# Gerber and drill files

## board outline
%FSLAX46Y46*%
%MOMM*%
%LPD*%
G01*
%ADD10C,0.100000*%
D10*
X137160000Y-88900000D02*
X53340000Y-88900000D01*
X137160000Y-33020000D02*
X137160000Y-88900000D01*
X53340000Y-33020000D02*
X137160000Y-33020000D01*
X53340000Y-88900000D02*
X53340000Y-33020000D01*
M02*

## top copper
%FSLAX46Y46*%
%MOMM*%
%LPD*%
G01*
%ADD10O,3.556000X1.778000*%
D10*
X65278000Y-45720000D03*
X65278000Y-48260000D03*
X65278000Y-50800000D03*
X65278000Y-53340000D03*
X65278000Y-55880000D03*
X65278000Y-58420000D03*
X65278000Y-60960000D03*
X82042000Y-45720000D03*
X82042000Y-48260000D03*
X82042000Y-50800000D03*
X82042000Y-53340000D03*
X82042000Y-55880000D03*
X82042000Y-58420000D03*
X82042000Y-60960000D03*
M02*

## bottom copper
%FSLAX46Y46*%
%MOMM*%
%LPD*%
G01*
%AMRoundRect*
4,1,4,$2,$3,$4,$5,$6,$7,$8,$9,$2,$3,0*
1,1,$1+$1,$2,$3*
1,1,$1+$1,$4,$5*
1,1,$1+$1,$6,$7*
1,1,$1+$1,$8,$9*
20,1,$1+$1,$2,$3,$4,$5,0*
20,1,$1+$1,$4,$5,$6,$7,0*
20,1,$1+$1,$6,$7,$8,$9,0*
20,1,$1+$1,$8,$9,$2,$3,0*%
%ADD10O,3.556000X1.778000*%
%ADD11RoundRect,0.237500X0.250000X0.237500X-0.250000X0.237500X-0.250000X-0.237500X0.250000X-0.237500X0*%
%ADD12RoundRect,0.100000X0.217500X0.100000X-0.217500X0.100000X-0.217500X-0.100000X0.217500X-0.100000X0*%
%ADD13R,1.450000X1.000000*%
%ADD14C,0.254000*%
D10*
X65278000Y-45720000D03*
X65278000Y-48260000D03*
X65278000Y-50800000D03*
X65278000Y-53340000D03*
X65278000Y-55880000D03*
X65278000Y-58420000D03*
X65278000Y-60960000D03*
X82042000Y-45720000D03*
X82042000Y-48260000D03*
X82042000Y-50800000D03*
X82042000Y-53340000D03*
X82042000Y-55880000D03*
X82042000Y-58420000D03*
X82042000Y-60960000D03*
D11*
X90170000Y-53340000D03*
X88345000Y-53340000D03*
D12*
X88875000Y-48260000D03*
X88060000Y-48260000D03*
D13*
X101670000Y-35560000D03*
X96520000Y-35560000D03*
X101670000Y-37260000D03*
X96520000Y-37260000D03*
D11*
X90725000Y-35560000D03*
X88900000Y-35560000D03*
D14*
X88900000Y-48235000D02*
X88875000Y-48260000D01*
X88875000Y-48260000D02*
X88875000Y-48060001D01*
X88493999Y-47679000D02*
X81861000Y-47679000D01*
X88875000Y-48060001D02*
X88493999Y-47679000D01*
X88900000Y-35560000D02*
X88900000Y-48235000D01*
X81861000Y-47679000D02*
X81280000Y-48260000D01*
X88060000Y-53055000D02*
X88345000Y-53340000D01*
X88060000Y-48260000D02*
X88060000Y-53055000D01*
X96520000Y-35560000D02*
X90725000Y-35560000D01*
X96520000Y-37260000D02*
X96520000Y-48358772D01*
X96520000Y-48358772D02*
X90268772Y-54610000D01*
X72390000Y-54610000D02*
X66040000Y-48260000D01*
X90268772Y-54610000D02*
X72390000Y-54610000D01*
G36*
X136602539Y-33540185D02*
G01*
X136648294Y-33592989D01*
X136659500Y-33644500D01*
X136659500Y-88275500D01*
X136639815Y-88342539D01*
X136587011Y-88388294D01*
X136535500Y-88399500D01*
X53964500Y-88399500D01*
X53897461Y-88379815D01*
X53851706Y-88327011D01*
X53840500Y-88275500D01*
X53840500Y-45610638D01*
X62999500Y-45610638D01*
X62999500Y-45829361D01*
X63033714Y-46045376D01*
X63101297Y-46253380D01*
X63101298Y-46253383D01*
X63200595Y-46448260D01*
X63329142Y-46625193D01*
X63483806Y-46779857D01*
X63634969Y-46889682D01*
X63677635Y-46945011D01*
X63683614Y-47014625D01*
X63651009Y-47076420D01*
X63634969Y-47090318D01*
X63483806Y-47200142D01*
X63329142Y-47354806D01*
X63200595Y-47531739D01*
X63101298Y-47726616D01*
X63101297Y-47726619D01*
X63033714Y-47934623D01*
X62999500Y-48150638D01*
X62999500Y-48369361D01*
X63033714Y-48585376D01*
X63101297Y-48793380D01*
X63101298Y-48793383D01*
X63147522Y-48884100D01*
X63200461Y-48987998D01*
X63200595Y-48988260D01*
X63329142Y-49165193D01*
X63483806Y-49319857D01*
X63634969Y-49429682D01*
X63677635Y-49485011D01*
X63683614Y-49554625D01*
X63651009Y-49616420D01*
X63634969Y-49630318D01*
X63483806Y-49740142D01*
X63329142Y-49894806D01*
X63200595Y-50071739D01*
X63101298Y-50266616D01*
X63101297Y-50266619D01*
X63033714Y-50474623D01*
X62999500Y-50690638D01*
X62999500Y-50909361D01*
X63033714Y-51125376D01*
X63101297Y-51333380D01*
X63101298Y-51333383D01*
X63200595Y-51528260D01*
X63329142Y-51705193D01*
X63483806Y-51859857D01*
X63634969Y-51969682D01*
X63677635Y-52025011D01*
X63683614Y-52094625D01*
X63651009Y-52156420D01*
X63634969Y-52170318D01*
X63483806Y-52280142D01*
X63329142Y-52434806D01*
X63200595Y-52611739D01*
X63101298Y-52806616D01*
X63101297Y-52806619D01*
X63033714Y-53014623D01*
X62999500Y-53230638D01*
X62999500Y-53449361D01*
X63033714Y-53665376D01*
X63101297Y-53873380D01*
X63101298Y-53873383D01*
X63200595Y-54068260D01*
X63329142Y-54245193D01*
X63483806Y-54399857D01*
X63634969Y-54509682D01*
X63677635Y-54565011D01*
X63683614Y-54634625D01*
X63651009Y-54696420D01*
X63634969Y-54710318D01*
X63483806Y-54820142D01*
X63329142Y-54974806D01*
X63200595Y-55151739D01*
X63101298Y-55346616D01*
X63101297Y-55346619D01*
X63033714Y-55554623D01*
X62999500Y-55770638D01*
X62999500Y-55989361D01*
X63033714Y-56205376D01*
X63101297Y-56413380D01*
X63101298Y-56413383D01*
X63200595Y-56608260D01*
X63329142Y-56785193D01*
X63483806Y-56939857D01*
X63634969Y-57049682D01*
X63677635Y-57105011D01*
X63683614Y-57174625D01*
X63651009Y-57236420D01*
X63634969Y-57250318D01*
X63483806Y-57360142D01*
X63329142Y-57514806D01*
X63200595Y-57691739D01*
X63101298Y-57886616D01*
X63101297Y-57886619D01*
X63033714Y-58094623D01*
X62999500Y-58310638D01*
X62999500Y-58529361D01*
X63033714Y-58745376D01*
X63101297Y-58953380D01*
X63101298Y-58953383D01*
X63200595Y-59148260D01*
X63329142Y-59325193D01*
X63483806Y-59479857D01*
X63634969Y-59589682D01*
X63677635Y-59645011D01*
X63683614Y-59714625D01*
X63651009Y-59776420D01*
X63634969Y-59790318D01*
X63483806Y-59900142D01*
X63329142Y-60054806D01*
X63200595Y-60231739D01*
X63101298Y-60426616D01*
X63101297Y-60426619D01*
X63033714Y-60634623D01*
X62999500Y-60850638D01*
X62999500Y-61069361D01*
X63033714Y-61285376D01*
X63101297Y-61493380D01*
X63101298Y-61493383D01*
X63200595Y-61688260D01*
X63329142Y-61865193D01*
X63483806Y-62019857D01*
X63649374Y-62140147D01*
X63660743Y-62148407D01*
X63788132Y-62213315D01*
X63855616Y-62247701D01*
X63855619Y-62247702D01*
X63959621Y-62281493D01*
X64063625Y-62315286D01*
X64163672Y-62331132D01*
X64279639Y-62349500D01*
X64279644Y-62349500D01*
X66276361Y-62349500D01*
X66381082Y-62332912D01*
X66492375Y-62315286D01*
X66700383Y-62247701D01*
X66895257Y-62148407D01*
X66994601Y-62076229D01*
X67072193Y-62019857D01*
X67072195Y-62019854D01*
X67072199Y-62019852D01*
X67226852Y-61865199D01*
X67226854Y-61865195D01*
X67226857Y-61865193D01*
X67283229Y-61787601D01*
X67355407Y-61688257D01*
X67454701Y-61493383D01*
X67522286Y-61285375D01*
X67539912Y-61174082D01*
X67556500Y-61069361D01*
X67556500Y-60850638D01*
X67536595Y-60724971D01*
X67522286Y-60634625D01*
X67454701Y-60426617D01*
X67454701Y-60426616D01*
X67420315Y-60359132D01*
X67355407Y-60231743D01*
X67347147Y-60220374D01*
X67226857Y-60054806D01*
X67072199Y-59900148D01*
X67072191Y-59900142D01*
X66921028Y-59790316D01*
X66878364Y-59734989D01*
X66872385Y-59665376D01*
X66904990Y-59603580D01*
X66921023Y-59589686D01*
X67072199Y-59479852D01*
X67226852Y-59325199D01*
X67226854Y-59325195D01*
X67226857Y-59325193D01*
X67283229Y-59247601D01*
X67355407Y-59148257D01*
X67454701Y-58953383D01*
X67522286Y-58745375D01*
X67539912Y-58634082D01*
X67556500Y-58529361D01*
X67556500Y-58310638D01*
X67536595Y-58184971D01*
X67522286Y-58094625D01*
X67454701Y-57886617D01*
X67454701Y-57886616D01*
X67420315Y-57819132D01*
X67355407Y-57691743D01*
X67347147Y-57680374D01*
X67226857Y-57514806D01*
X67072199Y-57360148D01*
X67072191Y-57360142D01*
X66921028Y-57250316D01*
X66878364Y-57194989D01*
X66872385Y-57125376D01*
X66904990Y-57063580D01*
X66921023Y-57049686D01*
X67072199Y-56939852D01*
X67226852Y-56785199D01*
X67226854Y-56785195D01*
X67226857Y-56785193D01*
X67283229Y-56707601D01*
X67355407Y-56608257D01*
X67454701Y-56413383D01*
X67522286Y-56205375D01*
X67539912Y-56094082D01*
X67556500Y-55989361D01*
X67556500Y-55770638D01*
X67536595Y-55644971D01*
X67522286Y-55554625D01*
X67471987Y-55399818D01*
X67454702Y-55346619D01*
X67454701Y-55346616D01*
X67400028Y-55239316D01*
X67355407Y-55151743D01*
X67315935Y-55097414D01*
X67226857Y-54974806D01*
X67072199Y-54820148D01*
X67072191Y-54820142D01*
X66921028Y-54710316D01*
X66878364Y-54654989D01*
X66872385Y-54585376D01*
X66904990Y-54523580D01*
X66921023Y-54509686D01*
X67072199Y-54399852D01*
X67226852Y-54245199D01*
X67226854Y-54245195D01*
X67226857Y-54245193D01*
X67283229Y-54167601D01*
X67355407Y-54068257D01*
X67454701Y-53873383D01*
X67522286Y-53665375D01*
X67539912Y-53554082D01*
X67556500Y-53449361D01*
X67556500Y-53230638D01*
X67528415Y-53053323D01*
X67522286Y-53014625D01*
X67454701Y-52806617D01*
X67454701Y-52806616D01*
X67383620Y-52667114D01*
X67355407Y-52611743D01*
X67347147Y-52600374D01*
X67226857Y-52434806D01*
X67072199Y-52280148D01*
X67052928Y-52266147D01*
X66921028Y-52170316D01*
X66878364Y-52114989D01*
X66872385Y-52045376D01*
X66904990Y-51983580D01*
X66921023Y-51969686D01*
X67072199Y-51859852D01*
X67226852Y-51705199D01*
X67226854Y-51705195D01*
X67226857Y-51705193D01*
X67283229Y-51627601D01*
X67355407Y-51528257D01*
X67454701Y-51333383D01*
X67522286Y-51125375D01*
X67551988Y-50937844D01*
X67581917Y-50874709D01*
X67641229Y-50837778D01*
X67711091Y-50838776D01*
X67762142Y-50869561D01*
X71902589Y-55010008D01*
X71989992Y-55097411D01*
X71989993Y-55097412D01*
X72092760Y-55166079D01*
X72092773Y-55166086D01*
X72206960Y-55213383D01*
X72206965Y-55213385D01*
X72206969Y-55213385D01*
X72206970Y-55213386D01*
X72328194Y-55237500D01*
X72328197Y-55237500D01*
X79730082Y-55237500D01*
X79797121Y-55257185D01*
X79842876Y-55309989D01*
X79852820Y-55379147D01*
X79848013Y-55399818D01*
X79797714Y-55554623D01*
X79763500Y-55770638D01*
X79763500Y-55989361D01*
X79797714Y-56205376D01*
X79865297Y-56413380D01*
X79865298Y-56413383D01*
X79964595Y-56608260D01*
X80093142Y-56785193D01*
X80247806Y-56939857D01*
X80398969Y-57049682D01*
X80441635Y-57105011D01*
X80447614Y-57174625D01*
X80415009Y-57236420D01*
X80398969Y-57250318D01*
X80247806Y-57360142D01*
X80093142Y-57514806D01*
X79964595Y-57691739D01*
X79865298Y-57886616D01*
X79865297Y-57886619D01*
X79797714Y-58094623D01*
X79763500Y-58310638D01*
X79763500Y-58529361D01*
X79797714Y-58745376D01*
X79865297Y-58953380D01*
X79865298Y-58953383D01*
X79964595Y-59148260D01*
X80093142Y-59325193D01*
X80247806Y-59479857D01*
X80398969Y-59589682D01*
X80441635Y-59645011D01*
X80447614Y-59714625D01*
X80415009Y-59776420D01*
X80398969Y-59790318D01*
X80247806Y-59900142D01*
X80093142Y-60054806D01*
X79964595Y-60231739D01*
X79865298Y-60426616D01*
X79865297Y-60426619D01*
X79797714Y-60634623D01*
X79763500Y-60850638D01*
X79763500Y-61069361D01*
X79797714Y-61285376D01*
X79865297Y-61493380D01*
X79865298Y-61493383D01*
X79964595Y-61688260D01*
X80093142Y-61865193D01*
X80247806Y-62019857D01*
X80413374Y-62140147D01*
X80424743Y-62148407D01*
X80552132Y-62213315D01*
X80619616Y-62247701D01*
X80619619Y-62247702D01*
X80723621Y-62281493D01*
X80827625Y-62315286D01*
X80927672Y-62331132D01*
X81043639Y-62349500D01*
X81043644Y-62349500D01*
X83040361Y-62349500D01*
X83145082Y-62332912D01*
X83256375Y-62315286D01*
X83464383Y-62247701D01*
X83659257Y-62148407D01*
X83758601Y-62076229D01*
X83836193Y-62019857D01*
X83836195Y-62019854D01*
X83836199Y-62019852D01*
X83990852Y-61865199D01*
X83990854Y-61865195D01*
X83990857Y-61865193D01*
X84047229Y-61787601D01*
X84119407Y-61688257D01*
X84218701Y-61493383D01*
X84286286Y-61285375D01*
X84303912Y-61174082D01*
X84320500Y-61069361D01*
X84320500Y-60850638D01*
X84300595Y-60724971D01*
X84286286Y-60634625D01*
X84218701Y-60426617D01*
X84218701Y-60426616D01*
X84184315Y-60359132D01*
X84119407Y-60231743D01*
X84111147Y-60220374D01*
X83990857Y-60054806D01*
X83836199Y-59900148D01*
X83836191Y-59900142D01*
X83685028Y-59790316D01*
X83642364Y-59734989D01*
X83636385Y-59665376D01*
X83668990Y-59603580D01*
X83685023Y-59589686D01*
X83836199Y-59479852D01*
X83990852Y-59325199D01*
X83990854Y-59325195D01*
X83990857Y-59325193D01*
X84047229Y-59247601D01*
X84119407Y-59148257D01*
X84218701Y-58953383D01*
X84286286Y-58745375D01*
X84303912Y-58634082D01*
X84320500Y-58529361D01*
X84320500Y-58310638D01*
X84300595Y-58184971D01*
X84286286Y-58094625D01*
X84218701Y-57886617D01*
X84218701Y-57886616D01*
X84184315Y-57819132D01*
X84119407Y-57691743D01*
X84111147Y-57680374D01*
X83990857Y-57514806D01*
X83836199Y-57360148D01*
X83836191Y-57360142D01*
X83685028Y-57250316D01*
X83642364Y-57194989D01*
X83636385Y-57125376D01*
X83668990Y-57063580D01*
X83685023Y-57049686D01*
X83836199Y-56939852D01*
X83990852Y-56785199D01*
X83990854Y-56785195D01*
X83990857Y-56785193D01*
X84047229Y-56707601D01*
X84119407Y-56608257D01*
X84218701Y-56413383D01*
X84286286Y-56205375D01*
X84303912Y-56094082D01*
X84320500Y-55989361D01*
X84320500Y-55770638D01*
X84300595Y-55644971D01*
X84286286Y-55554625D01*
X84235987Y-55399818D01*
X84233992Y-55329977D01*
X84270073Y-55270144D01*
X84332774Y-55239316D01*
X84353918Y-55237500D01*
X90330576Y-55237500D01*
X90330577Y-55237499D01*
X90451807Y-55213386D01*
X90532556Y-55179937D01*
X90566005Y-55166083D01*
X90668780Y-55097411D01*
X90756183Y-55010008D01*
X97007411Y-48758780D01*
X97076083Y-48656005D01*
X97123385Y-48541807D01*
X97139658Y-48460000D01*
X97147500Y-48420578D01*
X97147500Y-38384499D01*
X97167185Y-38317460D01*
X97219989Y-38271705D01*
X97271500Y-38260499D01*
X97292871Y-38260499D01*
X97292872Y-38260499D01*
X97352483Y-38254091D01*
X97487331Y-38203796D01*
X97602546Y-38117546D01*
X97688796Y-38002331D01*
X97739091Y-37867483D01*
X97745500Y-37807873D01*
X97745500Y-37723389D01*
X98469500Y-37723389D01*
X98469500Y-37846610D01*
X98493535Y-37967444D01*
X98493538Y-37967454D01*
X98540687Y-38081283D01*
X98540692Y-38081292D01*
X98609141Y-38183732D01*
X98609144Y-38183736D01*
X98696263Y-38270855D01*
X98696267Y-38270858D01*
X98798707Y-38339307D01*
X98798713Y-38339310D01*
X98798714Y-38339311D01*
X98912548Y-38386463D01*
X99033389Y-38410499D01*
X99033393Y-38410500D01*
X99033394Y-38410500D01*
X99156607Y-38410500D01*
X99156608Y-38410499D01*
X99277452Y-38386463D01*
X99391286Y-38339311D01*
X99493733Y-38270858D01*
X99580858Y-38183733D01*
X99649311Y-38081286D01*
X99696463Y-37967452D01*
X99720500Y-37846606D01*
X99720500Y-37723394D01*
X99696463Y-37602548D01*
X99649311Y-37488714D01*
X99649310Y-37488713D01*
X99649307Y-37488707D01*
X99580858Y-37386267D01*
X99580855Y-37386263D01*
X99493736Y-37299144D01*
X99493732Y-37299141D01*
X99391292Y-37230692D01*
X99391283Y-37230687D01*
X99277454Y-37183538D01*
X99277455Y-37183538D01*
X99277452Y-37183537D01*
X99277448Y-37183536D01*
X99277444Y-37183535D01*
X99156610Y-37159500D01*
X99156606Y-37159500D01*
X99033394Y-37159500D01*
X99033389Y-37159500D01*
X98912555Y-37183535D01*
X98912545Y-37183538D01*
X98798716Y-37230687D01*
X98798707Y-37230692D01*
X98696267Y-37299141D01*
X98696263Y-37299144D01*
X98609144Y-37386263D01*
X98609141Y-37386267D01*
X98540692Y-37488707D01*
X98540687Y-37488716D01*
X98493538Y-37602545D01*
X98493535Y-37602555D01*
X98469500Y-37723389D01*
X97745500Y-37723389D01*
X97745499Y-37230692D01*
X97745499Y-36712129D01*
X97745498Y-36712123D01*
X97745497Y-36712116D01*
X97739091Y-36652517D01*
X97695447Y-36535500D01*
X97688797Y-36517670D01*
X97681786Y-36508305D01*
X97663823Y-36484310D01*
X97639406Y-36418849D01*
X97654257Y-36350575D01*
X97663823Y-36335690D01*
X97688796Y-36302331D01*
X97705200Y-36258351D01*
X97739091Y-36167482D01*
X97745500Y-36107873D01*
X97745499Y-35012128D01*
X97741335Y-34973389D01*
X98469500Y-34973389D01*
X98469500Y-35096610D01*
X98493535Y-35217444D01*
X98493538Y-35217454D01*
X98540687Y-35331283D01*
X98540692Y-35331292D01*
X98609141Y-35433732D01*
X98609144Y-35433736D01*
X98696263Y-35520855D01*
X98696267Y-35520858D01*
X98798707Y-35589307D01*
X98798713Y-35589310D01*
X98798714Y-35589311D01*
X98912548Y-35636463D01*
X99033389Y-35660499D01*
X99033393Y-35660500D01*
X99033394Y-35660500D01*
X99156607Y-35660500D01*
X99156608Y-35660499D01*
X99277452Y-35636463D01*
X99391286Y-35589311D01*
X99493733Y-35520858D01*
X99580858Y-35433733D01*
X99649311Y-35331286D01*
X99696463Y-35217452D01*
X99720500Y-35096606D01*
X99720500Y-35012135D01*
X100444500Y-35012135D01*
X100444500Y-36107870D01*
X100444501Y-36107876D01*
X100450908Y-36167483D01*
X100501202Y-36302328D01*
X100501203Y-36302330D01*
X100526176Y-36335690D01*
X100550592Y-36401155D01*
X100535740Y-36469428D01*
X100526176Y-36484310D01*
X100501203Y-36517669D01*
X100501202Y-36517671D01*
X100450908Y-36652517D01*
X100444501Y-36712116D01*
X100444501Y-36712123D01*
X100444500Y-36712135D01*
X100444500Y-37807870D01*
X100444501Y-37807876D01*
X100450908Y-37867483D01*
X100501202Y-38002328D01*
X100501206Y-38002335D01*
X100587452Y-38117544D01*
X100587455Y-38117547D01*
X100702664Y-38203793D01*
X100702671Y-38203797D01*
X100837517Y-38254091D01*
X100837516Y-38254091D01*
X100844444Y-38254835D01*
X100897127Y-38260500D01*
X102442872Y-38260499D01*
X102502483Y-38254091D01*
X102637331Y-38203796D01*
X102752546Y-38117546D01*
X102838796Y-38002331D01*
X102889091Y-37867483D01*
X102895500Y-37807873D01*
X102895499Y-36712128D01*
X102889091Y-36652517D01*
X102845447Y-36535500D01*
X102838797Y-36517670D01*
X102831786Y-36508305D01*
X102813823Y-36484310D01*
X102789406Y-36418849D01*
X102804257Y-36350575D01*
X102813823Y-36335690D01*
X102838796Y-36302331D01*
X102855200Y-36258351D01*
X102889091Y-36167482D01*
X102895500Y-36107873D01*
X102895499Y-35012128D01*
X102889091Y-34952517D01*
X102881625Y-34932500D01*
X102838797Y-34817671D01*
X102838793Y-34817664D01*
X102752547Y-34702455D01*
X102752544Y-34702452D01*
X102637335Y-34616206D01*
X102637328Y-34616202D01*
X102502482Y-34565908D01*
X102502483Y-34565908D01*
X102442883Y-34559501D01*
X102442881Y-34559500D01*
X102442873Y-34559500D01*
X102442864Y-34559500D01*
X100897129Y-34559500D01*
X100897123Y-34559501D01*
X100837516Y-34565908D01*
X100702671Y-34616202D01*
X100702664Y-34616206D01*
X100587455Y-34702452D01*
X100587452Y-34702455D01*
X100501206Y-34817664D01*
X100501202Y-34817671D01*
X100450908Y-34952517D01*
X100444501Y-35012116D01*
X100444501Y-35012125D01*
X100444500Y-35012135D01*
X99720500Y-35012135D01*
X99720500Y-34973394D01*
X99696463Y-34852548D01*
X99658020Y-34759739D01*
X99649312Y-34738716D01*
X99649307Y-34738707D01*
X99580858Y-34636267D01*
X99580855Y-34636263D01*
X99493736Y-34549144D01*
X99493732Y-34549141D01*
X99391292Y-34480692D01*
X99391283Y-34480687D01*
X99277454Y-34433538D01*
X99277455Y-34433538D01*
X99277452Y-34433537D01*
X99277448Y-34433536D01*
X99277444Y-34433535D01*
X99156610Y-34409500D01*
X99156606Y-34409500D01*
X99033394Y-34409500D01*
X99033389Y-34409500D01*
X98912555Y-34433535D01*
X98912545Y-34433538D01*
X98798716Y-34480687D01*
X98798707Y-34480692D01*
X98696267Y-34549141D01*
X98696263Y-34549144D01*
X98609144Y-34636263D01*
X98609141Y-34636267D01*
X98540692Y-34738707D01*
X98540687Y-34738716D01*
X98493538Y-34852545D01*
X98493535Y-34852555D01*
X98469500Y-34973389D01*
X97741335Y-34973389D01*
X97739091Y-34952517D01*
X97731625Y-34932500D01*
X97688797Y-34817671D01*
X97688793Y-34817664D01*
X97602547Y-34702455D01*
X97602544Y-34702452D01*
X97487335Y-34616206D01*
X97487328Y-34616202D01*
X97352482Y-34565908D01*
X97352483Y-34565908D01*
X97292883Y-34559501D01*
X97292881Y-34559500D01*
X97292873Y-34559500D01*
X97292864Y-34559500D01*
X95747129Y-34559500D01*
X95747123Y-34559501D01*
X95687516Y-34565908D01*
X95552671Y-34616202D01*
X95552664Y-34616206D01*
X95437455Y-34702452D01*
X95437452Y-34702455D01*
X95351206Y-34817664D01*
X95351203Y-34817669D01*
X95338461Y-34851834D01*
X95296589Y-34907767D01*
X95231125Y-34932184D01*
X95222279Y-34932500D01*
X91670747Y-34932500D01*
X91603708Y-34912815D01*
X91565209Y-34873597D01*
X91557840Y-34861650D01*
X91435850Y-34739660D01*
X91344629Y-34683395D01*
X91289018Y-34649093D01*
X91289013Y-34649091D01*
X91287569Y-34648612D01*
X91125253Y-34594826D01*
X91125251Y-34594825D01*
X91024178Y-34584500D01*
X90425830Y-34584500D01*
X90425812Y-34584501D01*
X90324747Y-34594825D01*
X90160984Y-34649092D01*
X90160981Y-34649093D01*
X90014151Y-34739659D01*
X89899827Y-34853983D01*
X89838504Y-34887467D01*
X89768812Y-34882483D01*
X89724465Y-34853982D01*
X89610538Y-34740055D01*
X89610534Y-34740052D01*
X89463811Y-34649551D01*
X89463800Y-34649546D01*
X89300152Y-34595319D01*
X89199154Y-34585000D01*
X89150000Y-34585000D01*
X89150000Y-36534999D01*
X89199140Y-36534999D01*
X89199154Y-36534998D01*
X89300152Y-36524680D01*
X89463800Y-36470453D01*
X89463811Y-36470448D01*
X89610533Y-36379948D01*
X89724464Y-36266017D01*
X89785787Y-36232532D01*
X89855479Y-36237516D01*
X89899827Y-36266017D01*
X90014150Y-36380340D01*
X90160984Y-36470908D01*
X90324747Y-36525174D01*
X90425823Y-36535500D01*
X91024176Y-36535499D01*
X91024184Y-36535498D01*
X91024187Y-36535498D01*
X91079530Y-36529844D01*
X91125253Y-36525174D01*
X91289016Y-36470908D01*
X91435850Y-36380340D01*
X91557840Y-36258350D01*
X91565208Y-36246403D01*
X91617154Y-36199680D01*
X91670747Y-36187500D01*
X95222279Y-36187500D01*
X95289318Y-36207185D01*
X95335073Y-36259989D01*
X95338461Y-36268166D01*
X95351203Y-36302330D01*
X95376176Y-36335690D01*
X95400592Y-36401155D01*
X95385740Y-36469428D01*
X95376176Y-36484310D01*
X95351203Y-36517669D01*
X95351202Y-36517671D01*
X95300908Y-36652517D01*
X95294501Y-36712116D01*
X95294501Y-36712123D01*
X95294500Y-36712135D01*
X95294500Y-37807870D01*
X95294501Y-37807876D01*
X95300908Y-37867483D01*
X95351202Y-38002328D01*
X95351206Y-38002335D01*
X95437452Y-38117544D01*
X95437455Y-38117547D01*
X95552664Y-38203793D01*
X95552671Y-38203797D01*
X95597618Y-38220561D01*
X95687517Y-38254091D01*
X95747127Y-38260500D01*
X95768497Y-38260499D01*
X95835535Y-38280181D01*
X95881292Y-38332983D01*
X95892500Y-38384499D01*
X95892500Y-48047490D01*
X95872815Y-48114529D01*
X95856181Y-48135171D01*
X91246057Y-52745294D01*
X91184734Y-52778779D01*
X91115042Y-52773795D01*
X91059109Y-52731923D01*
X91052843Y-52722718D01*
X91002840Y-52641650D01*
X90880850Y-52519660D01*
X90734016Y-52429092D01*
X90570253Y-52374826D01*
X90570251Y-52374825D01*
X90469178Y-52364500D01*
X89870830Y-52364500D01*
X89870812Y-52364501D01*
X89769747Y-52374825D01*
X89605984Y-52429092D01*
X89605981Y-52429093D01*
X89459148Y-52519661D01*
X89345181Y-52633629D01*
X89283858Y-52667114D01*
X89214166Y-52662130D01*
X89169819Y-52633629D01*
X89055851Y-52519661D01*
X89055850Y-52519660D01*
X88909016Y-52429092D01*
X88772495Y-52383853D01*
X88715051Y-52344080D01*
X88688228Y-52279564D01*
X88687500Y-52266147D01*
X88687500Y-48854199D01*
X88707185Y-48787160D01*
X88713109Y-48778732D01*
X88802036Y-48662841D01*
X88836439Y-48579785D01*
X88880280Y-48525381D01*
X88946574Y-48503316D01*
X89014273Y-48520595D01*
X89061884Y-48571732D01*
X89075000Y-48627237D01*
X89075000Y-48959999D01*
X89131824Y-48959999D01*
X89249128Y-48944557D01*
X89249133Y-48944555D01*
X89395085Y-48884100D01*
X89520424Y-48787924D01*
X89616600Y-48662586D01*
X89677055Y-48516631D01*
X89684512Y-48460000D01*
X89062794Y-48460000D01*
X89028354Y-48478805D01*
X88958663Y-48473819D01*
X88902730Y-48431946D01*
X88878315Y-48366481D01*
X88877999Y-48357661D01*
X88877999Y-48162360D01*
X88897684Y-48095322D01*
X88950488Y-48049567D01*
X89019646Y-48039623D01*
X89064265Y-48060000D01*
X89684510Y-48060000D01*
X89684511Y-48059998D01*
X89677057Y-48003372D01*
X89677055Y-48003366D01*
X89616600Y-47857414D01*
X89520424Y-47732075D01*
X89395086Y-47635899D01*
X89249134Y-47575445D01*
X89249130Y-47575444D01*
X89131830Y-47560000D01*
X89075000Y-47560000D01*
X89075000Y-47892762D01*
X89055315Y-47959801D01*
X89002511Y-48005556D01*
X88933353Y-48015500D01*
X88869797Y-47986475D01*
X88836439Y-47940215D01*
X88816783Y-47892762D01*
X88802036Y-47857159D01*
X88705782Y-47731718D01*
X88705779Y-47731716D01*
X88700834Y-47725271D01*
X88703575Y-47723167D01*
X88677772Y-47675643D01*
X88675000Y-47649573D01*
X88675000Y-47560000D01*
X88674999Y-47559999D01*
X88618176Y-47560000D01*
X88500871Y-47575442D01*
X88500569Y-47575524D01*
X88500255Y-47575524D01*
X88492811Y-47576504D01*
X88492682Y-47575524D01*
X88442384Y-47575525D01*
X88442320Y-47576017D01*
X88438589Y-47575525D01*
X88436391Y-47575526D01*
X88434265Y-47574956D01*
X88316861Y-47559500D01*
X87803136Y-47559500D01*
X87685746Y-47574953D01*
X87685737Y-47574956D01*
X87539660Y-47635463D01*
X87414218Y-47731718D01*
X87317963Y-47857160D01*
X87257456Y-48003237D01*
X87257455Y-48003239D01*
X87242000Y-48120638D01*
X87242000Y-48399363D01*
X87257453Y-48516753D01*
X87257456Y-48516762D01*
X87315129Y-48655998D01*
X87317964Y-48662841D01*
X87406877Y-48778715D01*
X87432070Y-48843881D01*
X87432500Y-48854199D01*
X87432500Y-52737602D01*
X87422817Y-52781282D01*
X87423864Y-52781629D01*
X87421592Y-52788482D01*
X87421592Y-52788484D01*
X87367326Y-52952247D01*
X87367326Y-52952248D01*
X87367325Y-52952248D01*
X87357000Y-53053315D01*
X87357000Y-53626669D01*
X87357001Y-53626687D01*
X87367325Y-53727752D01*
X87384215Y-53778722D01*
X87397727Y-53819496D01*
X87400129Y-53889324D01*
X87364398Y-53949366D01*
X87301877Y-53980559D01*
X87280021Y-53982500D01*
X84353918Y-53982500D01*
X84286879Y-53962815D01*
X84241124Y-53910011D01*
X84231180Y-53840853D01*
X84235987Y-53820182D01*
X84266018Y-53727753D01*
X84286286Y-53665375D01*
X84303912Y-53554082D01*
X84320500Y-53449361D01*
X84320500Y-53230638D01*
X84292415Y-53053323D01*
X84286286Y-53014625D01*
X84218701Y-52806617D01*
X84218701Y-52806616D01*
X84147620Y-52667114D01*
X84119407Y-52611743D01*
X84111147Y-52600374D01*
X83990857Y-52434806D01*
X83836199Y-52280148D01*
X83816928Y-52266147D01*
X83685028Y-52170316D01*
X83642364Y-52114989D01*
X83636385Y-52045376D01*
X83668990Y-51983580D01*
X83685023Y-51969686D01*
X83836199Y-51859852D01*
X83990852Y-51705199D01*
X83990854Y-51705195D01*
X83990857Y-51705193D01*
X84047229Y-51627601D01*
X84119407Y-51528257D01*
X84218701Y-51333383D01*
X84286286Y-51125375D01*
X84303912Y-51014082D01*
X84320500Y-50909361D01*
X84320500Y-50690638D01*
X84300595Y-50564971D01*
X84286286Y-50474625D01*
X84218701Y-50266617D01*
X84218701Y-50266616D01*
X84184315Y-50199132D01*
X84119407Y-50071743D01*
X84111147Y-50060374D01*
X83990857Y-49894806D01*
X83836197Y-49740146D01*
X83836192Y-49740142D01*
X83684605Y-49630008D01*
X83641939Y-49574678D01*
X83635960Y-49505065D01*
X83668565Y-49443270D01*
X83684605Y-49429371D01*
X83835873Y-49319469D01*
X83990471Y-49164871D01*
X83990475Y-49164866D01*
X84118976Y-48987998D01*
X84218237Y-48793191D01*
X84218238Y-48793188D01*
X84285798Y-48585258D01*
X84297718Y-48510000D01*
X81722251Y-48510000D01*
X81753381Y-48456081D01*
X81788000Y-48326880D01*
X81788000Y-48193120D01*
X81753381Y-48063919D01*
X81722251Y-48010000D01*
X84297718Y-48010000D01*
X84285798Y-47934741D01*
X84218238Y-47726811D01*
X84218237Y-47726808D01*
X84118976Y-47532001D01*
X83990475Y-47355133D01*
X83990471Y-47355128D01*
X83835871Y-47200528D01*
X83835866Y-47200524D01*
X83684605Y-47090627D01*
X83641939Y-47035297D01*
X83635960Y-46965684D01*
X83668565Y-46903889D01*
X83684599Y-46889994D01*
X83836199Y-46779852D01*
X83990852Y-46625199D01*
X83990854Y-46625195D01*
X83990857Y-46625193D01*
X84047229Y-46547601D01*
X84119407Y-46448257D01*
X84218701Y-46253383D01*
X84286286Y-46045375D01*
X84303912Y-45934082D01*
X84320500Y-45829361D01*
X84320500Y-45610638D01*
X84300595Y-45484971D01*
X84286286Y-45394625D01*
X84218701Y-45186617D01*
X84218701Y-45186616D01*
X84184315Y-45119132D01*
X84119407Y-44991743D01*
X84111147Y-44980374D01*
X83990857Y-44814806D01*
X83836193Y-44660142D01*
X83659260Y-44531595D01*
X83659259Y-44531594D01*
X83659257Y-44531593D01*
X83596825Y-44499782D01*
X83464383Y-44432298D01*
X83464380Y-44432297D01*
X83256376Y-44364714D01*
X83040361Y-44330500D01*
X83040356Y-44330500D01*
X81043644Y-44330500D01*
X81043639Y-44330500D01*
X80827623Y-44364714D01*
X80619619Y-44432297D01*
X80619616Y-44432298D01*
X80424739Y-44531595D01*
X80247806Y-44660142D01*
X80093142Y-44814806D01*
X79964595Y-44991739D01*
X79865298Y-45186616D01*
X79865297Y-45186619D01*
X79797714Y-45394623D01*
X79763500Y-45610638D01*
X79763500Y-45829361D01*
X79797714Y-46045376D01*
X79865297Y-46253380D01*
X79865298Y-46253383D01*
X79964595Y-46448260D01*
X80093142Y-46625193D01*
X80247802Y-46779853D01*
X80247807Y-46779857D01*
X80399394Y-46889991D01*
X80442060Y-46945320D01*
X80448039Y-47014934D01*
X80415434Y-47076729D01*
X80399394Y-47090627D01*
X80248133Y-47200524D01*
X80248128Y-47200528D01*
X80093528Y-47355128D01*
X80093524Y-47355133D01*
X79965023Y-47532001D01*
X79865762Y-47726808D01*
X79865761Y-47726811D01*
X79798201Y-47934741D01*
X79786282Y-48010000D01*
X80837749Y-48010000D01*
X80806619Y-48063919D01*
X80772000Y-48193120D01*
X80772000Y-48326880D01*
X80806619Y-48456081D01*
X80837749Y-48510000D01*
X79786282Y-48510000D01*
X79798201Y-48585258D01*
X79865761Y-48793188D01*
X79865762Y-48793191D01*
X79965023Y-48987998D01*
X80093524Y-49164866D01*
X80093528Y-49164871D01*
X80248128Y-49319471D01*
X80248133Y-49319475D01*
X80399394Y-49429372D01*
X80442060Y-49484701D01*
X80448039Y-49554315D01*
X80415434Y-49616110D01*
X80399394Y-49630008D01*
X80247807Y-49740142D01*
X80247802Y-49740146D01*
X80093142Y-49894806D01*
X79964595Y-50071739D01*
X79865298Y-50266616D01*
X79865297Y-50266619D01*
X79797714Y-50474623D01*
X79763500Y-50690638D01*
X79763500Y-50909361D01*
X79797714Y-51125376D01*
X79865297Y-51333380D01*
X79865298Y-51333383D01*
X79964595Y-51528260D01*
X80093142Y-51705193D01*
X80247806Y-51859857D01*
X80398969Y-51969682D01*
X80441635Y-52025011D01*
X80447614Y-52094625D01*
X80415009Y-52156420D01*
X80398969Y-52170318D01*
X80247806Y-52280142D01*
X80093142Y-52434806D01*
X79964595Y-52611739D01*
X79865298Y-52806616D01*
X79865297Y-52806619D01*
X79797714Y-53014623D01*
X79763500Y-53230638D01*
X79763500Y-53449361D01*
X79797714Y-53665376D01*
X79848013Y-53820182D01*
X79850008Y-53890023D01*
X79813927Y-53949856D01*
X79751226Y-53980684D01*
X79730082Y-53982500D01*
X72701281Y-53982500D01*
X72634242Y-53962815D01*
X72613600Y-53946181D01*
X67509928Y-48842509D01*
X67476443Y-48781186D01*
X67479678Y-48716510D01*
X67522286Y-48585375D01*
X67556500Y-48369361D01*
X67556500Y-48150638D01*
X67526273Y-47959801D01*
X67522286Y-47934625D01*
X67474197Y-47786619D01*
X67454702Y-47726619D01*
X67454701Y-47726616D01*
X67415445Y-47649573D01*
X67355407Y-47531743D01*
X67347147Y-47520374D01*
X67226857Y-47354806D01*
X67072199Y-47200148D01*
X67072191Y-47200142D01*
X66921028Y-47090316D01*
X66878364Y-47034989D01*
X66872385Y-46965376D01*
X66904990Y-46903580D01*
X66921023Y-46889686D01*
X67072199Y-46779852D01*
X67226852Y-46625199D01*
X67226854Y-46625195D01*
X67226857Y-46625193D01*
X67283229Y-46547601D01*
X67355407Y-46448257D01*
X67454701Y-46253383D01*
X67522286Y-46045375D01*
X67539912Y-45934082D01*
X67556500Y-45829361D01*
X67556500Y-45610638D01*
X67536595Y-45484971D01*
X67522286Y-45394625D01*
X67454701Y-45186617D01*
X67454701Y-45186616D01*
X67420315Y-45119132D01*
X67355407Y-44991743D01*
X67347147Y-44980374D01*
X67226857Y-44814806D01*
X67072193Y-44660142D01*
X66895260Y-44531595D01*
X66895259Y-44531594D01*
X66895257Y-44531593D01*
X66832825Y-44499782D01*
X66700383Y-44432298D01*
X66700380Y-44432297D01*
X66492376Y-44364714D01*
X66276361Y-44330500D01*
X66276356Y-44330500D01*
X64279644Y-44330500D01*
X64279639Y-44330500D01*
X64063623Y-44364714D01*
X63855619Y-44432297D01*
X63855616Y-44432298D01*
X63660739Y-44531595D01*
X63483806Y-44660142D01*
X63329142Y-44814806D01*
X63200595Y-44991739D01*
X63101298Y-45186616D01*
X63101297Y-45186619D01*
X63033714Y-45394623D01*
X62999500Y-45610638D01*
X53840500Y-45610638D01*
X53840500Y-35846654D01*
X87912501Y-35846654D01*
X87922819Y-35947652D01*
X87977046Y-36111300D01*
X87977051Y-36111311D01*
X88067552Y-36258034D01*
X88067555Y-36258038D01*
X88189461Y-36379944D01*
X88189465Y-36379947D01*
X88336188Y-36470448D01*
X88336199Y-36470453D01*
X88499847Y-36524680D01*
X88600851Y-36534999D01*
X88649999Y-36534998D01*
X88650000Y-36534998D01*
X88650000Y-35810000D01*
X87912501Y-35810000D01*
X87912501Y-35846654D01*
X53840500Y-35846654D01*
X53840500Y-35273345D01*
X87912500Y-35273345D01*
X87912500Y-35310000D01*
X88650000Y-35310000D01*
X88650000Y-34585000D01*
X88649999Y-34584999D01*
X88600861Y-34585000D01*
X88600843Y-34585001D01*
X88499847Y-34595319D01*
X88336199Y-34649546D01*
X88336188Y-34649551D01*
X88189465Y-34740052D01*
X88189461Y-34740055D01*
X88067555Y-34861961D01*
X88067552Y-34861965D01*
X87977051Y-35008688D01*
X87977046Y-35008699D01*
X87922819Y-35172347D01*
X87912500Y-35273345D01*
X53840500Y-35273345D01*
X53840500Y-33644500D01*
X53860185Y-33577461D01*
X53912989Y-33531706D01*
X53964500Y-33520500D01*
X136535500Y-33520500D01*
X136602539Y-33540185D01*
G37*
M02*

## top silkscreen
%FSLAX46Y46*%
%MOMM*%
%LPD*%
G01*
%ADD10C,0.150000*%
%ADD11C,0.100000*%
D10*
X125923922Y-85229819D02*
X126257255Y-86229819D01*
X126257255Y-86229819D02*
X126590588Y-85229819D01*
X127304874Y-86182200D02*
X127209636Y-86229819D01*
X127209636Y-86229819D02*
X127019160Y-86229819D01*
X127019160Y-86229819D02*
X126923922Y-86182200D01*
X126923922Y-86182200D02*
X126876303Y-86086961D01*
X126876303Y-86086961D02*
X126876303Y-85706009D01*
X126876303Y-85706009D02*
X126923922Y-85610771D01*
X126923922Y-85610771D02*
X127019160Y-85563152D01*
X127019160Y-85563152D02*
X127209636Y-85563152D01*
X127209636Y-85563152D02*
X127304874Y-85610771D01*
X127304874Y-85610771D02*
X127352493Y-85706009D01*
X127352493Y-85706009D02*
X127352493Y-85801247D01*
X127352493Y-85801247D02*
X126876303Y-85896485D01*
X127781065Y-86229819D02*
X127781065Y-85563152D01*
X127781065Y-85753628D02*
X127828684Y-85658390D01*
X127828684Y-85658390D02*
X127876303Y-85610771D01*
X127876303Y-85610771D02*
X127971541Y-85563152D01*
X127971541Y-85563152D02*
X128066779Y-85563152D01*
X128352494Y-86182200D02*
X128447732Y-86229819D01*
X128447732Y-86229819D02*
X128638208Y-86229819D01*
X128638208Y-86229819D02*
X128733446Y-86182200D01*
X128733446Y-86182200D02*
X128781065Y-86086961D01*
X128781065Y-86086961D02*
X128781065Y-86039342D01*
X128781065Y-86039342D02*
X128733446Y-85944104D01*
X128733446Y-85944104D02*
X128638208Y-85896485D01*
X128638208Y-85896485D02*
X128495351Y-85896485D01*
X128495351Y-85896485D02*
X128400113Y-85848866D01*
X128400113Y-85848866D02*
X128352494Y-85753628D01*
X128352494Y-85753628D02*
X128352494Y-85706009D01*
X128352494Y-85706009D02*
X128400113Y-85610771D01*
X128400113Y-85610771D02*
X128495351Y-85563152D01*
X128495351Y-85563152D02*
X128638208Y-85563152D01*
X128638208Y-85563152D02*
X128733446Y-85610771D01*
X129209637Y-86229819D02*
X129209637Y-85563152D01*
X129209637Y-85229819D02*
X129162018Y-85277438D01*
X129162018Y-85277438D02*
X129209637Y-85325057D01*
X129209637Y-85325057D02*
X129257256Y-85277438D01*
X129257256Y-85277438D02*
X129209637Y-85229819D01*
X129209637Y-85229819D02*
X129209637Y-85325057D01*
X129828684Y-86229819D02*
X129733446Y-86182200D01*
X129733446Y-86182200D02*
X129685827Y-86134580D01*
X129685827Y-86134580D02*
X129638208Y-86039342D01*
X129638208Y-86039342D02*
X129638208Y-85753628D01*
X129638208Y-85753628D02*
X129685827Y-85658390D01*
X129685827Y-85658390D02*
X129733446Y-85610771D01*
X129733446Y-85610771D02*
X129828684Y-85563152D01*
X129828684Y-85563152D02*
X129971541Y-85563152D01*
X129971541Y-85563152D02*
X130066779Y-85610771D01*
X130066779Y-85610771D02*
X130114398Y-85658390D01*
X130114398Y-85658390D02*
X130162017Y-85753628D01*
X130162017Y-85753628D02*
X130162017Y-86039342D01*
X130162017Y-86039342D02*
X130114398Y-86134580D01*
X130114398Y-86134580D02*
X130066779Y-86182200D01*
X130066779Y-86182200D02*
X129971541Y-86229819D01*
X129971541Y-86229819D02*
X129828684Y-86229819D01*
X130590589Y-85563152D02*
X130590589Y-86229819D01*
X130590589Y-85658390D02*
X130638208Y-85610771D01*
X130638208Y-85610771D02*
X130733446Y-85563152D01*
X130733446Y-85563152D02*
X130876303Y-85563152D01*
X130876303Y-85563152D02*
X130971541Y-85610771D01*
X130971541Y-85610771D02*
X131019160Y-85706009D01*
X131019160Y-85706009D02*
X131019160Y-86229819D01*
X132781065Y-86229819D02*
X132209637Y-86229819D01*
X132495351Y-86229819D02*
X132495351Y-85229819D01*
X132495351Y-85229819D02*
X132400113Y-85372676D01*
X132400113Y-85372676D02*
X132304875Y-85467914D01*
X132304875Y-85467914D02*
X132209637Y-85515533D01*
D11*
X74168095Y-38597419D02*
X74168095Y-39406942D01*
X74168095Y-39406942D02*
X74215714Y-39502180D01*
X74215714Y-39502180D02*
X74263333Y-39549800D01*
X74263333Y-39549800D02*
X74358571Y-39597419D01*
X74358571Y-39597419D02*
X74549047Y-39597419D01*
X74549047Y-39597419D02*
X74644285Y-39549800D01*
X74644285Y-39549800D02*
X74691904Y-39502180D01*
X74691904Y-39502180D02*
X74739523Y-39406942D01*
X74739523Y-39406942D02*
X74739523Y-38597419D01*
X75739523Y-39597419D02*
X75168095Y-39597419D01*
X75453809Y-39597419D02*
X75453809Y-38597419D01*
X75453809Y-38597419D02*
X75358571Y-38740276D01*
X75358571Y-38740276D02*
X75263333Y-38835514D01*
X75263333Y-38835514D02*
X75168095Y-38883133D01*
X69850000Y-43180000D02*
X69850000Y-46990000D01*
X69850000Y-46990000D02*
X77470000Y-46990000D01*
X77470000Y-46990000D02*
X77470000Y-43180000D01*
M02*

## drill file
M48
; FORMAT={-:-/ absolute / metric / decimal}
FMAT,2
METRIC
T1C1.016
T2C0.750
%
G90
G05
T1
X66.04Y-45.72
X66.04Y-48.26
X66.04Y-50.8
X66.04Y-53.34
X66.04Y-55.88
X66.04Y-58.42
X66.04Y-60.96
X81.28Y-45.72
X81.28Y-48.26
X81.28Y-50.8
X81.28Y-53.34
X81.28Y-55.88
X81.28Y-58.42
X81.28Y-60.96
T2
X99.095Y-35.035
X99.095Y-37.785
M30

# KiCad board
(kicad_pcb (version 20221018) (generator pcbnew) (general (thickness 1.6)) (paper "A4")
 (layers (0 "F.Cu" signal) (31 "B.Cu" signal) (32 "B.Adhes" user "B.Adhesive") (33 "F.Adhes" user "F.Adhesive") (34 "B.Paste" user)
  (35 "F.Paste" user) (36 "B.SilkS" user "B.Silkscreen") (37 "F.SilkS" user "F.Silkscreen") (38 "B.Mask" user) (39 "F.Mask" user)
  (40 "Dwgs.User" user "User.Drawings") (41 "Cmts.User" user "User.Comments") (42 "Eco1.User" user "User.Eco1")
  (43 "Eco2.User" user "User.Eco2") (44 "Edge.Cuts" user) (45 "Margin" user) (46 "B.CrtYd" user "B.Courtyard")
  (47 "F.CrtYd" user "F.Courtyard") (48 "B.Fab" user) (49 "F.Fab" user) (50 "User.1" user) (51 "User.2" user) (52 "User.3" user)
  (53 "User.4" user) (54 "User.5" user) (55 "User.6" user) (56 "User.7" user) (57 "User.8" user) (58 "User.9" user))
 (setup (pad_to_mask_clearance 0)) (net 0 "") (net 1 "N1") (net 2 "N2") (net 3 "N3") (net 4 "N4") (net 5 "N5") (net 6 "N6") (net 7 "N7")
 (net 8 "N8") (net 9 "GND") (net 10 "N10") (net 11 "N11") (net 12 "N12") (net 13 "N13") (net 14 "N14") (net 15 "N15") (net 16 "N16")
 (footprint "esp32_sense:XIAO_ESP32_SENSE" (layer "F.Cu") (at 73.66 53.34)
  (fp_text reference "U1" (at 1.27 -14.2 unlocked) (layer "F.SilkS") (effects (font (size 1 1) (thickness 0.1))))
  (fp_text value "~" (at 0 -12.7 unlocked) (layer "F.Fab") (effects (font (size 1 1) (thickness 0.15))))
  (fp_line (start -3.81 -10.16) (end -3.81 -6.35) (stroke (width 0.1) (type default)) (layer "F.SilkS"))
  (fp_line (start -3.81 -6.35) (end 3.81 -6.35) (stroke (width 0.1) (type default)) (layer "F.SilkS"))
  (fp_line (start 3.81 -6.35) (end 3.81 -10.16) (stroke (width 0.1) (type default)) (layer "F.SilkS"))
  (pad "1" thru_hole oval (at -7.62 -7.62) (size 3.556 1.778) (drill 1.016 (offset -0.762 0)) (layers "*.Cu" "*.Mask") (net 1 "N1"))
  (pad "2" thru_hole oval (at -7.62 -5.08) (size 3.556 1.778) (drill 1.016 (offset -0.762 0)) (layers "*.Cu" "*.Mask") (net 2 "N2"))
  (pad "3" thru_hole oval (at -7.62 -2.54) (size 3.556 1.778) (drill 1.016 (offset -0.762 0)) (layers "*.Cu" "*.Mask") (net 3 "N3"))
  (pad "4" thru_hole oval (at -7.62 0) (size 3.556 1.778) (drill 1.016 (offset -0.762 0)) (layers "*.Cu" "*.Mask") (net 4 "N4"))
  (pad "5" thru_hole oval (at -7.62 2.54) (size 3.556 1.778) (drill 1.016 (offset -0.762 0)) (layers "*.Cu" "*.Mask") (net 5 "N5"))
  (pad "6" thru_hole oval (at -7.62 5.08) (size 3.556 1.778) (drill 1.016 (offset -0.762 0)) (layers "*.Cu" "*.Mask") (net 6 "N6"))
  (pad "7" thru_hole oval (at -7.62 7.62) (size 3.556 1.778) (drill 1.016 (offset -0.762 0)) (layers "*.Cu" "*.Mask") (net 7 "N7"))
  (pad "8" thru_hole oval (at 7.62 -7.62) (size 3.556 1.778) (drill 1.016 (offset 0.762 0)) (layers "*.Cu" "*.Mask") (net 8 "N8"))
  (pad "9" thru_hole oval (at 7.62 -5.08) (size 3.556 1.778) (drill 1.016 (offset 0.762 0)) (layers "*.Cu" "*.Mask") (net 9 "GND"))
  (pad "10" thru_hole oval (at 7.62 -2.54) (size 3.556 1.778) (drill 1.016 (offset 0.762 0)) (layers "*.Cu" "*.Mask") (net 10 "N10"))
  (pad "11" thru_hole oval (at 7.62 0) (size 3.556 1.778) (drill 1.016 (offset 0.762 0)) (layers "*.Cu" "*.Mask") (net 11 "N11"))
  (pad "12" thru_hole oval (at 7.62 2.54) (size 3.556 1.778) (drill 1.016 (offset 0.762 0)) (layers "*.Cu" "*.Mask") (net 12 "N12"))
  (pad "13" thru_hole oval (at 7.62 5.08) (size 3.556 1.778) (drill 1.016 (offset 0.762 0)) (layers "*.Cu" "*.Mask") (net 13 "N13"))
  (pad "14" thru_hole oval (at 7.62 7.62) (size 3.556 1.778) (drill 1.016 (offset 0.762 0)) (layers "*.Cu" "*.Mask") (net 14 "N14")))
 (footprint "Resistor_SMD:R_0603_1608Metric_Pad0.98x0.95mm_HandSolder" (layer "B.Cu") (at 89.2575 53.34 180)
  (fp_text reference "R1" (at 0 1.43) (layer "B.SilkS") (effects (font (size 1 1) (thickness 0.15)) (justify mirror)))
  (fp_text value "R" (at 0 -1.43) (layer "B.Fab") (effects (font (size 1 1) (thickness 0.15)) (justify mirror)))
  (pad "1" smd roundrect (at -0.9125 0 180) (size 0.975 0.95) (layers "B.Cu" "B.Paste" "B.Mask") (roundrect_rratio 0.25) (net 11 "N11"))
  (pad "2" smd roundrect (at 0.9125 0 180) (size 0.975 0.95) (layers "B.Cu" "B.Paste" "B.Mask") (roundrect_rratio 0.25) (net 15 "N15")))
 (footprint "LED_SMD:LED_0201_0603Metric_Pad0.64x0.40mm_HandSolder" (layer "B.Cu") (at 88.4675 48.26 180)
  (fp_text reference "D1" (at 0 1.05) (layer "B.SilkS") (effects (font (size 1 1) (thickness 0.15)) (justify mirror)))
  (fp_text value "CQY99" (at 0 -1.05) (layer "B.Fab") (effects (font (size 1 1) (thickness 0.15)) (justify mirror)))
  (pad "" smd roundrect (at -0.4325 0 180) (size 0.458 0.36) (layers "B.Paste") (roundrect_rratio 0.25))
  (pad "" smd roundrect (at 0.4325 0 180) (size 0.458 0.36) (layers "B.Paste") (roundrect_rratio 0.25))
  (pad "1" smd roundrect (at -0.4075 0 180) (size 0.635 0.4) (layers "B.Cu" "B.Mask") (roundrect_rratio 0.25) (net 9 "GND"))
  (pad "2" smd roundrect (at 0.4075 0 180) (size 0.635 0.4) (layers "B.Cu" "B.Mask") (roundrect_rratio 0.25) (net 15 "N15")))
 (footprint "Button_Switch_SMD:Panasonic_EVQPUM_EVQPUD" (layer "B.Cu") (at 99.095 36.41 180)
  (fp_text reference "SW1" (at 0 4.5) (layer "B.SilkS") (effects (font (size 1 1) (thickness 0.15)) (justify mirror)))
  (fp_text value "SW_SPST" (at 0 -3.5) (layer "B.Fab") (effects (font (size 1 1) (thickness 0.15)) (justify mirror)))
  (pad "" np_thru_hole circle (at 0 -1.375) (size 0.75 0.75) (drill 0.75) (layers "*.Cu" "*.Mask"))
  (pad "" np_thru_hole circle (at 0 1.375) (size 0.75 0.75) (drill 0.75) (layers "*.Cu" "*.Mask"))
  (pad "1" smd rect (at -2.575 0.85) (size 1.45 1) (layers "B.Cu" "B.Paste" "B.Mask") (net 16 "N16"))
  (pad "1" smd rect (at 2.575 0.85) (size 1.45 1) (layers "B.Cu" "B.Paste" "B.Mask") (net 16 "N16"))
  (pad "2" smd rect (at -2.575 -0.85) (size 1.45 1) (layers "B.Cu" "B.Paste" "B.Mask") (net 2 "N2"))
  (pad "2" smd rect (at 2.575 -0.85) (size 1.45 1) (layers "B.Cu" "B.Paste" "B.Mask") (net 2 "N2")))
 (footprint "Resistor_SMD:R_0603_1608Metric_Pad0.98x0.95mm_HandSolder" (layer "B.Cu") (at 89.8125 35.56 180)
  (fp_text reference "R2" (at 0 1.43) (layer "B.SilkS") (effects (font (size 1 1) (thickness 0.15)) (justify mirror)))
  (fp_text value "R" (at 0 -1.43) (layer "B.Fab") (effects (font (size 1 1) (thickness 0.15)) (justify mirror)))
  (pad "1" smd roundrect (at -0.9125 0 180) (size 0.975 0.95) (layers "B.Cu" "B.Paste" "B.Mask") (roundrect_rratio 0.25) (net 16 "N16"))
  (pad "2" smd roundrect (at 0.9125 0 180) (size 0.975 0.95) (layers "B.Cu" "B.Paste" "B.Mask") (roundrect_rratio 0.25) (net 9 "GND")))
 (gr_line (start 137.16 88.9) (end 53.34 88.9) (stroke (width 0.1) (type default)) (layer "Edge.Cuts"))
 (gr_line (start 137.16 33.02) (end 137.16 88.9) (stroke (width 0.1) (type default)) (layer "Edge.Cuts"))
 (gr_line (start 53.34 33.02) (end 137.16 33.02) (stroke (width 0.1) (type default)) (layer "Edge.Cuts"))
 (gr_line (start 53.34 88.9) (end 53.34 33.02) (stroke (width 0.1) (type default)) (layer "Edge.Cuts"))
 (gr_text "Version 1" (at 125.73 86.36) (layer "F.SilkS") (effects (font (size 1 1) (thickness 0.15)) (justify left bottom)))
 (segment (start 88.9 48.235) (end 88.875 48.26) (width 0.254) (layer "B.Cu") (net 9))
 (segment (start 88.875 48.26) (end 88.875 48.060001) (width 0.254) (layer "B.Cu") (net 9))
 (segment (start 88.493999 47.679) (end 81.861 47.679) (width 0.254) (layer "B.Cu") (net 9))
 (segment (start 88.875 48.060001) (end 88.493999 47.679) (width 0.254) (layer "B.Cu") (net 9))
 (segment (start 88.9 35.56) (end 88.9 48.235) (width 0.254) (layer "B.Cu") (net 9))
 (segment (start 81.861 47.679) (end 81.28 48.26) (width 0.254) (layer "B.Cu") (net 9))
 (segment (start 88.06 53.055) (end 88.345 53.34) (width 0.254) (layer "B.Cu") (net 15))
 (segment (start 88.06 48.26) (end 88.06 53.055) (width 0.254) (layer "B.Cu") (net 15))
 (segment (start 96.52 35.56) (end 90.725 35.56) (width 0.254) (layer "B.Cu") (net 16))
 (segment (start 96.52 37.26) (end 96.52 48.358772) (width 0.254) (layer "B.Cu") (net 2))
 (segment (start 96.52 48.358772) (end 90.268772 54.61) (width 0.254) (layer "B.Cu") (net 2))
 (segment (start 72.39 54.61) (end 66.04 48.26) (width 0.254) (layer "B.Cu") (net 2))
 (segment (start 90.268772 54.61) (end 72.39 54.61) (width 0.254) (layer "B.Cu") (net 2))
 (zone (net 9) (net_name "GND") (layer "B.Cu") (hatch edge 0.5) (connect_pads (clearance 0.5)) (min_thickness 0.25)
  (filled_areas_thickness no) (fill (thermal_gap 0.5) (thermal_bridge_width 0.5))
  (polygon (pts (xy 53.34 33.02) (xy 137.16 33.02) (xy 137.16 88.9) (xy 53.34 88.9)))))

